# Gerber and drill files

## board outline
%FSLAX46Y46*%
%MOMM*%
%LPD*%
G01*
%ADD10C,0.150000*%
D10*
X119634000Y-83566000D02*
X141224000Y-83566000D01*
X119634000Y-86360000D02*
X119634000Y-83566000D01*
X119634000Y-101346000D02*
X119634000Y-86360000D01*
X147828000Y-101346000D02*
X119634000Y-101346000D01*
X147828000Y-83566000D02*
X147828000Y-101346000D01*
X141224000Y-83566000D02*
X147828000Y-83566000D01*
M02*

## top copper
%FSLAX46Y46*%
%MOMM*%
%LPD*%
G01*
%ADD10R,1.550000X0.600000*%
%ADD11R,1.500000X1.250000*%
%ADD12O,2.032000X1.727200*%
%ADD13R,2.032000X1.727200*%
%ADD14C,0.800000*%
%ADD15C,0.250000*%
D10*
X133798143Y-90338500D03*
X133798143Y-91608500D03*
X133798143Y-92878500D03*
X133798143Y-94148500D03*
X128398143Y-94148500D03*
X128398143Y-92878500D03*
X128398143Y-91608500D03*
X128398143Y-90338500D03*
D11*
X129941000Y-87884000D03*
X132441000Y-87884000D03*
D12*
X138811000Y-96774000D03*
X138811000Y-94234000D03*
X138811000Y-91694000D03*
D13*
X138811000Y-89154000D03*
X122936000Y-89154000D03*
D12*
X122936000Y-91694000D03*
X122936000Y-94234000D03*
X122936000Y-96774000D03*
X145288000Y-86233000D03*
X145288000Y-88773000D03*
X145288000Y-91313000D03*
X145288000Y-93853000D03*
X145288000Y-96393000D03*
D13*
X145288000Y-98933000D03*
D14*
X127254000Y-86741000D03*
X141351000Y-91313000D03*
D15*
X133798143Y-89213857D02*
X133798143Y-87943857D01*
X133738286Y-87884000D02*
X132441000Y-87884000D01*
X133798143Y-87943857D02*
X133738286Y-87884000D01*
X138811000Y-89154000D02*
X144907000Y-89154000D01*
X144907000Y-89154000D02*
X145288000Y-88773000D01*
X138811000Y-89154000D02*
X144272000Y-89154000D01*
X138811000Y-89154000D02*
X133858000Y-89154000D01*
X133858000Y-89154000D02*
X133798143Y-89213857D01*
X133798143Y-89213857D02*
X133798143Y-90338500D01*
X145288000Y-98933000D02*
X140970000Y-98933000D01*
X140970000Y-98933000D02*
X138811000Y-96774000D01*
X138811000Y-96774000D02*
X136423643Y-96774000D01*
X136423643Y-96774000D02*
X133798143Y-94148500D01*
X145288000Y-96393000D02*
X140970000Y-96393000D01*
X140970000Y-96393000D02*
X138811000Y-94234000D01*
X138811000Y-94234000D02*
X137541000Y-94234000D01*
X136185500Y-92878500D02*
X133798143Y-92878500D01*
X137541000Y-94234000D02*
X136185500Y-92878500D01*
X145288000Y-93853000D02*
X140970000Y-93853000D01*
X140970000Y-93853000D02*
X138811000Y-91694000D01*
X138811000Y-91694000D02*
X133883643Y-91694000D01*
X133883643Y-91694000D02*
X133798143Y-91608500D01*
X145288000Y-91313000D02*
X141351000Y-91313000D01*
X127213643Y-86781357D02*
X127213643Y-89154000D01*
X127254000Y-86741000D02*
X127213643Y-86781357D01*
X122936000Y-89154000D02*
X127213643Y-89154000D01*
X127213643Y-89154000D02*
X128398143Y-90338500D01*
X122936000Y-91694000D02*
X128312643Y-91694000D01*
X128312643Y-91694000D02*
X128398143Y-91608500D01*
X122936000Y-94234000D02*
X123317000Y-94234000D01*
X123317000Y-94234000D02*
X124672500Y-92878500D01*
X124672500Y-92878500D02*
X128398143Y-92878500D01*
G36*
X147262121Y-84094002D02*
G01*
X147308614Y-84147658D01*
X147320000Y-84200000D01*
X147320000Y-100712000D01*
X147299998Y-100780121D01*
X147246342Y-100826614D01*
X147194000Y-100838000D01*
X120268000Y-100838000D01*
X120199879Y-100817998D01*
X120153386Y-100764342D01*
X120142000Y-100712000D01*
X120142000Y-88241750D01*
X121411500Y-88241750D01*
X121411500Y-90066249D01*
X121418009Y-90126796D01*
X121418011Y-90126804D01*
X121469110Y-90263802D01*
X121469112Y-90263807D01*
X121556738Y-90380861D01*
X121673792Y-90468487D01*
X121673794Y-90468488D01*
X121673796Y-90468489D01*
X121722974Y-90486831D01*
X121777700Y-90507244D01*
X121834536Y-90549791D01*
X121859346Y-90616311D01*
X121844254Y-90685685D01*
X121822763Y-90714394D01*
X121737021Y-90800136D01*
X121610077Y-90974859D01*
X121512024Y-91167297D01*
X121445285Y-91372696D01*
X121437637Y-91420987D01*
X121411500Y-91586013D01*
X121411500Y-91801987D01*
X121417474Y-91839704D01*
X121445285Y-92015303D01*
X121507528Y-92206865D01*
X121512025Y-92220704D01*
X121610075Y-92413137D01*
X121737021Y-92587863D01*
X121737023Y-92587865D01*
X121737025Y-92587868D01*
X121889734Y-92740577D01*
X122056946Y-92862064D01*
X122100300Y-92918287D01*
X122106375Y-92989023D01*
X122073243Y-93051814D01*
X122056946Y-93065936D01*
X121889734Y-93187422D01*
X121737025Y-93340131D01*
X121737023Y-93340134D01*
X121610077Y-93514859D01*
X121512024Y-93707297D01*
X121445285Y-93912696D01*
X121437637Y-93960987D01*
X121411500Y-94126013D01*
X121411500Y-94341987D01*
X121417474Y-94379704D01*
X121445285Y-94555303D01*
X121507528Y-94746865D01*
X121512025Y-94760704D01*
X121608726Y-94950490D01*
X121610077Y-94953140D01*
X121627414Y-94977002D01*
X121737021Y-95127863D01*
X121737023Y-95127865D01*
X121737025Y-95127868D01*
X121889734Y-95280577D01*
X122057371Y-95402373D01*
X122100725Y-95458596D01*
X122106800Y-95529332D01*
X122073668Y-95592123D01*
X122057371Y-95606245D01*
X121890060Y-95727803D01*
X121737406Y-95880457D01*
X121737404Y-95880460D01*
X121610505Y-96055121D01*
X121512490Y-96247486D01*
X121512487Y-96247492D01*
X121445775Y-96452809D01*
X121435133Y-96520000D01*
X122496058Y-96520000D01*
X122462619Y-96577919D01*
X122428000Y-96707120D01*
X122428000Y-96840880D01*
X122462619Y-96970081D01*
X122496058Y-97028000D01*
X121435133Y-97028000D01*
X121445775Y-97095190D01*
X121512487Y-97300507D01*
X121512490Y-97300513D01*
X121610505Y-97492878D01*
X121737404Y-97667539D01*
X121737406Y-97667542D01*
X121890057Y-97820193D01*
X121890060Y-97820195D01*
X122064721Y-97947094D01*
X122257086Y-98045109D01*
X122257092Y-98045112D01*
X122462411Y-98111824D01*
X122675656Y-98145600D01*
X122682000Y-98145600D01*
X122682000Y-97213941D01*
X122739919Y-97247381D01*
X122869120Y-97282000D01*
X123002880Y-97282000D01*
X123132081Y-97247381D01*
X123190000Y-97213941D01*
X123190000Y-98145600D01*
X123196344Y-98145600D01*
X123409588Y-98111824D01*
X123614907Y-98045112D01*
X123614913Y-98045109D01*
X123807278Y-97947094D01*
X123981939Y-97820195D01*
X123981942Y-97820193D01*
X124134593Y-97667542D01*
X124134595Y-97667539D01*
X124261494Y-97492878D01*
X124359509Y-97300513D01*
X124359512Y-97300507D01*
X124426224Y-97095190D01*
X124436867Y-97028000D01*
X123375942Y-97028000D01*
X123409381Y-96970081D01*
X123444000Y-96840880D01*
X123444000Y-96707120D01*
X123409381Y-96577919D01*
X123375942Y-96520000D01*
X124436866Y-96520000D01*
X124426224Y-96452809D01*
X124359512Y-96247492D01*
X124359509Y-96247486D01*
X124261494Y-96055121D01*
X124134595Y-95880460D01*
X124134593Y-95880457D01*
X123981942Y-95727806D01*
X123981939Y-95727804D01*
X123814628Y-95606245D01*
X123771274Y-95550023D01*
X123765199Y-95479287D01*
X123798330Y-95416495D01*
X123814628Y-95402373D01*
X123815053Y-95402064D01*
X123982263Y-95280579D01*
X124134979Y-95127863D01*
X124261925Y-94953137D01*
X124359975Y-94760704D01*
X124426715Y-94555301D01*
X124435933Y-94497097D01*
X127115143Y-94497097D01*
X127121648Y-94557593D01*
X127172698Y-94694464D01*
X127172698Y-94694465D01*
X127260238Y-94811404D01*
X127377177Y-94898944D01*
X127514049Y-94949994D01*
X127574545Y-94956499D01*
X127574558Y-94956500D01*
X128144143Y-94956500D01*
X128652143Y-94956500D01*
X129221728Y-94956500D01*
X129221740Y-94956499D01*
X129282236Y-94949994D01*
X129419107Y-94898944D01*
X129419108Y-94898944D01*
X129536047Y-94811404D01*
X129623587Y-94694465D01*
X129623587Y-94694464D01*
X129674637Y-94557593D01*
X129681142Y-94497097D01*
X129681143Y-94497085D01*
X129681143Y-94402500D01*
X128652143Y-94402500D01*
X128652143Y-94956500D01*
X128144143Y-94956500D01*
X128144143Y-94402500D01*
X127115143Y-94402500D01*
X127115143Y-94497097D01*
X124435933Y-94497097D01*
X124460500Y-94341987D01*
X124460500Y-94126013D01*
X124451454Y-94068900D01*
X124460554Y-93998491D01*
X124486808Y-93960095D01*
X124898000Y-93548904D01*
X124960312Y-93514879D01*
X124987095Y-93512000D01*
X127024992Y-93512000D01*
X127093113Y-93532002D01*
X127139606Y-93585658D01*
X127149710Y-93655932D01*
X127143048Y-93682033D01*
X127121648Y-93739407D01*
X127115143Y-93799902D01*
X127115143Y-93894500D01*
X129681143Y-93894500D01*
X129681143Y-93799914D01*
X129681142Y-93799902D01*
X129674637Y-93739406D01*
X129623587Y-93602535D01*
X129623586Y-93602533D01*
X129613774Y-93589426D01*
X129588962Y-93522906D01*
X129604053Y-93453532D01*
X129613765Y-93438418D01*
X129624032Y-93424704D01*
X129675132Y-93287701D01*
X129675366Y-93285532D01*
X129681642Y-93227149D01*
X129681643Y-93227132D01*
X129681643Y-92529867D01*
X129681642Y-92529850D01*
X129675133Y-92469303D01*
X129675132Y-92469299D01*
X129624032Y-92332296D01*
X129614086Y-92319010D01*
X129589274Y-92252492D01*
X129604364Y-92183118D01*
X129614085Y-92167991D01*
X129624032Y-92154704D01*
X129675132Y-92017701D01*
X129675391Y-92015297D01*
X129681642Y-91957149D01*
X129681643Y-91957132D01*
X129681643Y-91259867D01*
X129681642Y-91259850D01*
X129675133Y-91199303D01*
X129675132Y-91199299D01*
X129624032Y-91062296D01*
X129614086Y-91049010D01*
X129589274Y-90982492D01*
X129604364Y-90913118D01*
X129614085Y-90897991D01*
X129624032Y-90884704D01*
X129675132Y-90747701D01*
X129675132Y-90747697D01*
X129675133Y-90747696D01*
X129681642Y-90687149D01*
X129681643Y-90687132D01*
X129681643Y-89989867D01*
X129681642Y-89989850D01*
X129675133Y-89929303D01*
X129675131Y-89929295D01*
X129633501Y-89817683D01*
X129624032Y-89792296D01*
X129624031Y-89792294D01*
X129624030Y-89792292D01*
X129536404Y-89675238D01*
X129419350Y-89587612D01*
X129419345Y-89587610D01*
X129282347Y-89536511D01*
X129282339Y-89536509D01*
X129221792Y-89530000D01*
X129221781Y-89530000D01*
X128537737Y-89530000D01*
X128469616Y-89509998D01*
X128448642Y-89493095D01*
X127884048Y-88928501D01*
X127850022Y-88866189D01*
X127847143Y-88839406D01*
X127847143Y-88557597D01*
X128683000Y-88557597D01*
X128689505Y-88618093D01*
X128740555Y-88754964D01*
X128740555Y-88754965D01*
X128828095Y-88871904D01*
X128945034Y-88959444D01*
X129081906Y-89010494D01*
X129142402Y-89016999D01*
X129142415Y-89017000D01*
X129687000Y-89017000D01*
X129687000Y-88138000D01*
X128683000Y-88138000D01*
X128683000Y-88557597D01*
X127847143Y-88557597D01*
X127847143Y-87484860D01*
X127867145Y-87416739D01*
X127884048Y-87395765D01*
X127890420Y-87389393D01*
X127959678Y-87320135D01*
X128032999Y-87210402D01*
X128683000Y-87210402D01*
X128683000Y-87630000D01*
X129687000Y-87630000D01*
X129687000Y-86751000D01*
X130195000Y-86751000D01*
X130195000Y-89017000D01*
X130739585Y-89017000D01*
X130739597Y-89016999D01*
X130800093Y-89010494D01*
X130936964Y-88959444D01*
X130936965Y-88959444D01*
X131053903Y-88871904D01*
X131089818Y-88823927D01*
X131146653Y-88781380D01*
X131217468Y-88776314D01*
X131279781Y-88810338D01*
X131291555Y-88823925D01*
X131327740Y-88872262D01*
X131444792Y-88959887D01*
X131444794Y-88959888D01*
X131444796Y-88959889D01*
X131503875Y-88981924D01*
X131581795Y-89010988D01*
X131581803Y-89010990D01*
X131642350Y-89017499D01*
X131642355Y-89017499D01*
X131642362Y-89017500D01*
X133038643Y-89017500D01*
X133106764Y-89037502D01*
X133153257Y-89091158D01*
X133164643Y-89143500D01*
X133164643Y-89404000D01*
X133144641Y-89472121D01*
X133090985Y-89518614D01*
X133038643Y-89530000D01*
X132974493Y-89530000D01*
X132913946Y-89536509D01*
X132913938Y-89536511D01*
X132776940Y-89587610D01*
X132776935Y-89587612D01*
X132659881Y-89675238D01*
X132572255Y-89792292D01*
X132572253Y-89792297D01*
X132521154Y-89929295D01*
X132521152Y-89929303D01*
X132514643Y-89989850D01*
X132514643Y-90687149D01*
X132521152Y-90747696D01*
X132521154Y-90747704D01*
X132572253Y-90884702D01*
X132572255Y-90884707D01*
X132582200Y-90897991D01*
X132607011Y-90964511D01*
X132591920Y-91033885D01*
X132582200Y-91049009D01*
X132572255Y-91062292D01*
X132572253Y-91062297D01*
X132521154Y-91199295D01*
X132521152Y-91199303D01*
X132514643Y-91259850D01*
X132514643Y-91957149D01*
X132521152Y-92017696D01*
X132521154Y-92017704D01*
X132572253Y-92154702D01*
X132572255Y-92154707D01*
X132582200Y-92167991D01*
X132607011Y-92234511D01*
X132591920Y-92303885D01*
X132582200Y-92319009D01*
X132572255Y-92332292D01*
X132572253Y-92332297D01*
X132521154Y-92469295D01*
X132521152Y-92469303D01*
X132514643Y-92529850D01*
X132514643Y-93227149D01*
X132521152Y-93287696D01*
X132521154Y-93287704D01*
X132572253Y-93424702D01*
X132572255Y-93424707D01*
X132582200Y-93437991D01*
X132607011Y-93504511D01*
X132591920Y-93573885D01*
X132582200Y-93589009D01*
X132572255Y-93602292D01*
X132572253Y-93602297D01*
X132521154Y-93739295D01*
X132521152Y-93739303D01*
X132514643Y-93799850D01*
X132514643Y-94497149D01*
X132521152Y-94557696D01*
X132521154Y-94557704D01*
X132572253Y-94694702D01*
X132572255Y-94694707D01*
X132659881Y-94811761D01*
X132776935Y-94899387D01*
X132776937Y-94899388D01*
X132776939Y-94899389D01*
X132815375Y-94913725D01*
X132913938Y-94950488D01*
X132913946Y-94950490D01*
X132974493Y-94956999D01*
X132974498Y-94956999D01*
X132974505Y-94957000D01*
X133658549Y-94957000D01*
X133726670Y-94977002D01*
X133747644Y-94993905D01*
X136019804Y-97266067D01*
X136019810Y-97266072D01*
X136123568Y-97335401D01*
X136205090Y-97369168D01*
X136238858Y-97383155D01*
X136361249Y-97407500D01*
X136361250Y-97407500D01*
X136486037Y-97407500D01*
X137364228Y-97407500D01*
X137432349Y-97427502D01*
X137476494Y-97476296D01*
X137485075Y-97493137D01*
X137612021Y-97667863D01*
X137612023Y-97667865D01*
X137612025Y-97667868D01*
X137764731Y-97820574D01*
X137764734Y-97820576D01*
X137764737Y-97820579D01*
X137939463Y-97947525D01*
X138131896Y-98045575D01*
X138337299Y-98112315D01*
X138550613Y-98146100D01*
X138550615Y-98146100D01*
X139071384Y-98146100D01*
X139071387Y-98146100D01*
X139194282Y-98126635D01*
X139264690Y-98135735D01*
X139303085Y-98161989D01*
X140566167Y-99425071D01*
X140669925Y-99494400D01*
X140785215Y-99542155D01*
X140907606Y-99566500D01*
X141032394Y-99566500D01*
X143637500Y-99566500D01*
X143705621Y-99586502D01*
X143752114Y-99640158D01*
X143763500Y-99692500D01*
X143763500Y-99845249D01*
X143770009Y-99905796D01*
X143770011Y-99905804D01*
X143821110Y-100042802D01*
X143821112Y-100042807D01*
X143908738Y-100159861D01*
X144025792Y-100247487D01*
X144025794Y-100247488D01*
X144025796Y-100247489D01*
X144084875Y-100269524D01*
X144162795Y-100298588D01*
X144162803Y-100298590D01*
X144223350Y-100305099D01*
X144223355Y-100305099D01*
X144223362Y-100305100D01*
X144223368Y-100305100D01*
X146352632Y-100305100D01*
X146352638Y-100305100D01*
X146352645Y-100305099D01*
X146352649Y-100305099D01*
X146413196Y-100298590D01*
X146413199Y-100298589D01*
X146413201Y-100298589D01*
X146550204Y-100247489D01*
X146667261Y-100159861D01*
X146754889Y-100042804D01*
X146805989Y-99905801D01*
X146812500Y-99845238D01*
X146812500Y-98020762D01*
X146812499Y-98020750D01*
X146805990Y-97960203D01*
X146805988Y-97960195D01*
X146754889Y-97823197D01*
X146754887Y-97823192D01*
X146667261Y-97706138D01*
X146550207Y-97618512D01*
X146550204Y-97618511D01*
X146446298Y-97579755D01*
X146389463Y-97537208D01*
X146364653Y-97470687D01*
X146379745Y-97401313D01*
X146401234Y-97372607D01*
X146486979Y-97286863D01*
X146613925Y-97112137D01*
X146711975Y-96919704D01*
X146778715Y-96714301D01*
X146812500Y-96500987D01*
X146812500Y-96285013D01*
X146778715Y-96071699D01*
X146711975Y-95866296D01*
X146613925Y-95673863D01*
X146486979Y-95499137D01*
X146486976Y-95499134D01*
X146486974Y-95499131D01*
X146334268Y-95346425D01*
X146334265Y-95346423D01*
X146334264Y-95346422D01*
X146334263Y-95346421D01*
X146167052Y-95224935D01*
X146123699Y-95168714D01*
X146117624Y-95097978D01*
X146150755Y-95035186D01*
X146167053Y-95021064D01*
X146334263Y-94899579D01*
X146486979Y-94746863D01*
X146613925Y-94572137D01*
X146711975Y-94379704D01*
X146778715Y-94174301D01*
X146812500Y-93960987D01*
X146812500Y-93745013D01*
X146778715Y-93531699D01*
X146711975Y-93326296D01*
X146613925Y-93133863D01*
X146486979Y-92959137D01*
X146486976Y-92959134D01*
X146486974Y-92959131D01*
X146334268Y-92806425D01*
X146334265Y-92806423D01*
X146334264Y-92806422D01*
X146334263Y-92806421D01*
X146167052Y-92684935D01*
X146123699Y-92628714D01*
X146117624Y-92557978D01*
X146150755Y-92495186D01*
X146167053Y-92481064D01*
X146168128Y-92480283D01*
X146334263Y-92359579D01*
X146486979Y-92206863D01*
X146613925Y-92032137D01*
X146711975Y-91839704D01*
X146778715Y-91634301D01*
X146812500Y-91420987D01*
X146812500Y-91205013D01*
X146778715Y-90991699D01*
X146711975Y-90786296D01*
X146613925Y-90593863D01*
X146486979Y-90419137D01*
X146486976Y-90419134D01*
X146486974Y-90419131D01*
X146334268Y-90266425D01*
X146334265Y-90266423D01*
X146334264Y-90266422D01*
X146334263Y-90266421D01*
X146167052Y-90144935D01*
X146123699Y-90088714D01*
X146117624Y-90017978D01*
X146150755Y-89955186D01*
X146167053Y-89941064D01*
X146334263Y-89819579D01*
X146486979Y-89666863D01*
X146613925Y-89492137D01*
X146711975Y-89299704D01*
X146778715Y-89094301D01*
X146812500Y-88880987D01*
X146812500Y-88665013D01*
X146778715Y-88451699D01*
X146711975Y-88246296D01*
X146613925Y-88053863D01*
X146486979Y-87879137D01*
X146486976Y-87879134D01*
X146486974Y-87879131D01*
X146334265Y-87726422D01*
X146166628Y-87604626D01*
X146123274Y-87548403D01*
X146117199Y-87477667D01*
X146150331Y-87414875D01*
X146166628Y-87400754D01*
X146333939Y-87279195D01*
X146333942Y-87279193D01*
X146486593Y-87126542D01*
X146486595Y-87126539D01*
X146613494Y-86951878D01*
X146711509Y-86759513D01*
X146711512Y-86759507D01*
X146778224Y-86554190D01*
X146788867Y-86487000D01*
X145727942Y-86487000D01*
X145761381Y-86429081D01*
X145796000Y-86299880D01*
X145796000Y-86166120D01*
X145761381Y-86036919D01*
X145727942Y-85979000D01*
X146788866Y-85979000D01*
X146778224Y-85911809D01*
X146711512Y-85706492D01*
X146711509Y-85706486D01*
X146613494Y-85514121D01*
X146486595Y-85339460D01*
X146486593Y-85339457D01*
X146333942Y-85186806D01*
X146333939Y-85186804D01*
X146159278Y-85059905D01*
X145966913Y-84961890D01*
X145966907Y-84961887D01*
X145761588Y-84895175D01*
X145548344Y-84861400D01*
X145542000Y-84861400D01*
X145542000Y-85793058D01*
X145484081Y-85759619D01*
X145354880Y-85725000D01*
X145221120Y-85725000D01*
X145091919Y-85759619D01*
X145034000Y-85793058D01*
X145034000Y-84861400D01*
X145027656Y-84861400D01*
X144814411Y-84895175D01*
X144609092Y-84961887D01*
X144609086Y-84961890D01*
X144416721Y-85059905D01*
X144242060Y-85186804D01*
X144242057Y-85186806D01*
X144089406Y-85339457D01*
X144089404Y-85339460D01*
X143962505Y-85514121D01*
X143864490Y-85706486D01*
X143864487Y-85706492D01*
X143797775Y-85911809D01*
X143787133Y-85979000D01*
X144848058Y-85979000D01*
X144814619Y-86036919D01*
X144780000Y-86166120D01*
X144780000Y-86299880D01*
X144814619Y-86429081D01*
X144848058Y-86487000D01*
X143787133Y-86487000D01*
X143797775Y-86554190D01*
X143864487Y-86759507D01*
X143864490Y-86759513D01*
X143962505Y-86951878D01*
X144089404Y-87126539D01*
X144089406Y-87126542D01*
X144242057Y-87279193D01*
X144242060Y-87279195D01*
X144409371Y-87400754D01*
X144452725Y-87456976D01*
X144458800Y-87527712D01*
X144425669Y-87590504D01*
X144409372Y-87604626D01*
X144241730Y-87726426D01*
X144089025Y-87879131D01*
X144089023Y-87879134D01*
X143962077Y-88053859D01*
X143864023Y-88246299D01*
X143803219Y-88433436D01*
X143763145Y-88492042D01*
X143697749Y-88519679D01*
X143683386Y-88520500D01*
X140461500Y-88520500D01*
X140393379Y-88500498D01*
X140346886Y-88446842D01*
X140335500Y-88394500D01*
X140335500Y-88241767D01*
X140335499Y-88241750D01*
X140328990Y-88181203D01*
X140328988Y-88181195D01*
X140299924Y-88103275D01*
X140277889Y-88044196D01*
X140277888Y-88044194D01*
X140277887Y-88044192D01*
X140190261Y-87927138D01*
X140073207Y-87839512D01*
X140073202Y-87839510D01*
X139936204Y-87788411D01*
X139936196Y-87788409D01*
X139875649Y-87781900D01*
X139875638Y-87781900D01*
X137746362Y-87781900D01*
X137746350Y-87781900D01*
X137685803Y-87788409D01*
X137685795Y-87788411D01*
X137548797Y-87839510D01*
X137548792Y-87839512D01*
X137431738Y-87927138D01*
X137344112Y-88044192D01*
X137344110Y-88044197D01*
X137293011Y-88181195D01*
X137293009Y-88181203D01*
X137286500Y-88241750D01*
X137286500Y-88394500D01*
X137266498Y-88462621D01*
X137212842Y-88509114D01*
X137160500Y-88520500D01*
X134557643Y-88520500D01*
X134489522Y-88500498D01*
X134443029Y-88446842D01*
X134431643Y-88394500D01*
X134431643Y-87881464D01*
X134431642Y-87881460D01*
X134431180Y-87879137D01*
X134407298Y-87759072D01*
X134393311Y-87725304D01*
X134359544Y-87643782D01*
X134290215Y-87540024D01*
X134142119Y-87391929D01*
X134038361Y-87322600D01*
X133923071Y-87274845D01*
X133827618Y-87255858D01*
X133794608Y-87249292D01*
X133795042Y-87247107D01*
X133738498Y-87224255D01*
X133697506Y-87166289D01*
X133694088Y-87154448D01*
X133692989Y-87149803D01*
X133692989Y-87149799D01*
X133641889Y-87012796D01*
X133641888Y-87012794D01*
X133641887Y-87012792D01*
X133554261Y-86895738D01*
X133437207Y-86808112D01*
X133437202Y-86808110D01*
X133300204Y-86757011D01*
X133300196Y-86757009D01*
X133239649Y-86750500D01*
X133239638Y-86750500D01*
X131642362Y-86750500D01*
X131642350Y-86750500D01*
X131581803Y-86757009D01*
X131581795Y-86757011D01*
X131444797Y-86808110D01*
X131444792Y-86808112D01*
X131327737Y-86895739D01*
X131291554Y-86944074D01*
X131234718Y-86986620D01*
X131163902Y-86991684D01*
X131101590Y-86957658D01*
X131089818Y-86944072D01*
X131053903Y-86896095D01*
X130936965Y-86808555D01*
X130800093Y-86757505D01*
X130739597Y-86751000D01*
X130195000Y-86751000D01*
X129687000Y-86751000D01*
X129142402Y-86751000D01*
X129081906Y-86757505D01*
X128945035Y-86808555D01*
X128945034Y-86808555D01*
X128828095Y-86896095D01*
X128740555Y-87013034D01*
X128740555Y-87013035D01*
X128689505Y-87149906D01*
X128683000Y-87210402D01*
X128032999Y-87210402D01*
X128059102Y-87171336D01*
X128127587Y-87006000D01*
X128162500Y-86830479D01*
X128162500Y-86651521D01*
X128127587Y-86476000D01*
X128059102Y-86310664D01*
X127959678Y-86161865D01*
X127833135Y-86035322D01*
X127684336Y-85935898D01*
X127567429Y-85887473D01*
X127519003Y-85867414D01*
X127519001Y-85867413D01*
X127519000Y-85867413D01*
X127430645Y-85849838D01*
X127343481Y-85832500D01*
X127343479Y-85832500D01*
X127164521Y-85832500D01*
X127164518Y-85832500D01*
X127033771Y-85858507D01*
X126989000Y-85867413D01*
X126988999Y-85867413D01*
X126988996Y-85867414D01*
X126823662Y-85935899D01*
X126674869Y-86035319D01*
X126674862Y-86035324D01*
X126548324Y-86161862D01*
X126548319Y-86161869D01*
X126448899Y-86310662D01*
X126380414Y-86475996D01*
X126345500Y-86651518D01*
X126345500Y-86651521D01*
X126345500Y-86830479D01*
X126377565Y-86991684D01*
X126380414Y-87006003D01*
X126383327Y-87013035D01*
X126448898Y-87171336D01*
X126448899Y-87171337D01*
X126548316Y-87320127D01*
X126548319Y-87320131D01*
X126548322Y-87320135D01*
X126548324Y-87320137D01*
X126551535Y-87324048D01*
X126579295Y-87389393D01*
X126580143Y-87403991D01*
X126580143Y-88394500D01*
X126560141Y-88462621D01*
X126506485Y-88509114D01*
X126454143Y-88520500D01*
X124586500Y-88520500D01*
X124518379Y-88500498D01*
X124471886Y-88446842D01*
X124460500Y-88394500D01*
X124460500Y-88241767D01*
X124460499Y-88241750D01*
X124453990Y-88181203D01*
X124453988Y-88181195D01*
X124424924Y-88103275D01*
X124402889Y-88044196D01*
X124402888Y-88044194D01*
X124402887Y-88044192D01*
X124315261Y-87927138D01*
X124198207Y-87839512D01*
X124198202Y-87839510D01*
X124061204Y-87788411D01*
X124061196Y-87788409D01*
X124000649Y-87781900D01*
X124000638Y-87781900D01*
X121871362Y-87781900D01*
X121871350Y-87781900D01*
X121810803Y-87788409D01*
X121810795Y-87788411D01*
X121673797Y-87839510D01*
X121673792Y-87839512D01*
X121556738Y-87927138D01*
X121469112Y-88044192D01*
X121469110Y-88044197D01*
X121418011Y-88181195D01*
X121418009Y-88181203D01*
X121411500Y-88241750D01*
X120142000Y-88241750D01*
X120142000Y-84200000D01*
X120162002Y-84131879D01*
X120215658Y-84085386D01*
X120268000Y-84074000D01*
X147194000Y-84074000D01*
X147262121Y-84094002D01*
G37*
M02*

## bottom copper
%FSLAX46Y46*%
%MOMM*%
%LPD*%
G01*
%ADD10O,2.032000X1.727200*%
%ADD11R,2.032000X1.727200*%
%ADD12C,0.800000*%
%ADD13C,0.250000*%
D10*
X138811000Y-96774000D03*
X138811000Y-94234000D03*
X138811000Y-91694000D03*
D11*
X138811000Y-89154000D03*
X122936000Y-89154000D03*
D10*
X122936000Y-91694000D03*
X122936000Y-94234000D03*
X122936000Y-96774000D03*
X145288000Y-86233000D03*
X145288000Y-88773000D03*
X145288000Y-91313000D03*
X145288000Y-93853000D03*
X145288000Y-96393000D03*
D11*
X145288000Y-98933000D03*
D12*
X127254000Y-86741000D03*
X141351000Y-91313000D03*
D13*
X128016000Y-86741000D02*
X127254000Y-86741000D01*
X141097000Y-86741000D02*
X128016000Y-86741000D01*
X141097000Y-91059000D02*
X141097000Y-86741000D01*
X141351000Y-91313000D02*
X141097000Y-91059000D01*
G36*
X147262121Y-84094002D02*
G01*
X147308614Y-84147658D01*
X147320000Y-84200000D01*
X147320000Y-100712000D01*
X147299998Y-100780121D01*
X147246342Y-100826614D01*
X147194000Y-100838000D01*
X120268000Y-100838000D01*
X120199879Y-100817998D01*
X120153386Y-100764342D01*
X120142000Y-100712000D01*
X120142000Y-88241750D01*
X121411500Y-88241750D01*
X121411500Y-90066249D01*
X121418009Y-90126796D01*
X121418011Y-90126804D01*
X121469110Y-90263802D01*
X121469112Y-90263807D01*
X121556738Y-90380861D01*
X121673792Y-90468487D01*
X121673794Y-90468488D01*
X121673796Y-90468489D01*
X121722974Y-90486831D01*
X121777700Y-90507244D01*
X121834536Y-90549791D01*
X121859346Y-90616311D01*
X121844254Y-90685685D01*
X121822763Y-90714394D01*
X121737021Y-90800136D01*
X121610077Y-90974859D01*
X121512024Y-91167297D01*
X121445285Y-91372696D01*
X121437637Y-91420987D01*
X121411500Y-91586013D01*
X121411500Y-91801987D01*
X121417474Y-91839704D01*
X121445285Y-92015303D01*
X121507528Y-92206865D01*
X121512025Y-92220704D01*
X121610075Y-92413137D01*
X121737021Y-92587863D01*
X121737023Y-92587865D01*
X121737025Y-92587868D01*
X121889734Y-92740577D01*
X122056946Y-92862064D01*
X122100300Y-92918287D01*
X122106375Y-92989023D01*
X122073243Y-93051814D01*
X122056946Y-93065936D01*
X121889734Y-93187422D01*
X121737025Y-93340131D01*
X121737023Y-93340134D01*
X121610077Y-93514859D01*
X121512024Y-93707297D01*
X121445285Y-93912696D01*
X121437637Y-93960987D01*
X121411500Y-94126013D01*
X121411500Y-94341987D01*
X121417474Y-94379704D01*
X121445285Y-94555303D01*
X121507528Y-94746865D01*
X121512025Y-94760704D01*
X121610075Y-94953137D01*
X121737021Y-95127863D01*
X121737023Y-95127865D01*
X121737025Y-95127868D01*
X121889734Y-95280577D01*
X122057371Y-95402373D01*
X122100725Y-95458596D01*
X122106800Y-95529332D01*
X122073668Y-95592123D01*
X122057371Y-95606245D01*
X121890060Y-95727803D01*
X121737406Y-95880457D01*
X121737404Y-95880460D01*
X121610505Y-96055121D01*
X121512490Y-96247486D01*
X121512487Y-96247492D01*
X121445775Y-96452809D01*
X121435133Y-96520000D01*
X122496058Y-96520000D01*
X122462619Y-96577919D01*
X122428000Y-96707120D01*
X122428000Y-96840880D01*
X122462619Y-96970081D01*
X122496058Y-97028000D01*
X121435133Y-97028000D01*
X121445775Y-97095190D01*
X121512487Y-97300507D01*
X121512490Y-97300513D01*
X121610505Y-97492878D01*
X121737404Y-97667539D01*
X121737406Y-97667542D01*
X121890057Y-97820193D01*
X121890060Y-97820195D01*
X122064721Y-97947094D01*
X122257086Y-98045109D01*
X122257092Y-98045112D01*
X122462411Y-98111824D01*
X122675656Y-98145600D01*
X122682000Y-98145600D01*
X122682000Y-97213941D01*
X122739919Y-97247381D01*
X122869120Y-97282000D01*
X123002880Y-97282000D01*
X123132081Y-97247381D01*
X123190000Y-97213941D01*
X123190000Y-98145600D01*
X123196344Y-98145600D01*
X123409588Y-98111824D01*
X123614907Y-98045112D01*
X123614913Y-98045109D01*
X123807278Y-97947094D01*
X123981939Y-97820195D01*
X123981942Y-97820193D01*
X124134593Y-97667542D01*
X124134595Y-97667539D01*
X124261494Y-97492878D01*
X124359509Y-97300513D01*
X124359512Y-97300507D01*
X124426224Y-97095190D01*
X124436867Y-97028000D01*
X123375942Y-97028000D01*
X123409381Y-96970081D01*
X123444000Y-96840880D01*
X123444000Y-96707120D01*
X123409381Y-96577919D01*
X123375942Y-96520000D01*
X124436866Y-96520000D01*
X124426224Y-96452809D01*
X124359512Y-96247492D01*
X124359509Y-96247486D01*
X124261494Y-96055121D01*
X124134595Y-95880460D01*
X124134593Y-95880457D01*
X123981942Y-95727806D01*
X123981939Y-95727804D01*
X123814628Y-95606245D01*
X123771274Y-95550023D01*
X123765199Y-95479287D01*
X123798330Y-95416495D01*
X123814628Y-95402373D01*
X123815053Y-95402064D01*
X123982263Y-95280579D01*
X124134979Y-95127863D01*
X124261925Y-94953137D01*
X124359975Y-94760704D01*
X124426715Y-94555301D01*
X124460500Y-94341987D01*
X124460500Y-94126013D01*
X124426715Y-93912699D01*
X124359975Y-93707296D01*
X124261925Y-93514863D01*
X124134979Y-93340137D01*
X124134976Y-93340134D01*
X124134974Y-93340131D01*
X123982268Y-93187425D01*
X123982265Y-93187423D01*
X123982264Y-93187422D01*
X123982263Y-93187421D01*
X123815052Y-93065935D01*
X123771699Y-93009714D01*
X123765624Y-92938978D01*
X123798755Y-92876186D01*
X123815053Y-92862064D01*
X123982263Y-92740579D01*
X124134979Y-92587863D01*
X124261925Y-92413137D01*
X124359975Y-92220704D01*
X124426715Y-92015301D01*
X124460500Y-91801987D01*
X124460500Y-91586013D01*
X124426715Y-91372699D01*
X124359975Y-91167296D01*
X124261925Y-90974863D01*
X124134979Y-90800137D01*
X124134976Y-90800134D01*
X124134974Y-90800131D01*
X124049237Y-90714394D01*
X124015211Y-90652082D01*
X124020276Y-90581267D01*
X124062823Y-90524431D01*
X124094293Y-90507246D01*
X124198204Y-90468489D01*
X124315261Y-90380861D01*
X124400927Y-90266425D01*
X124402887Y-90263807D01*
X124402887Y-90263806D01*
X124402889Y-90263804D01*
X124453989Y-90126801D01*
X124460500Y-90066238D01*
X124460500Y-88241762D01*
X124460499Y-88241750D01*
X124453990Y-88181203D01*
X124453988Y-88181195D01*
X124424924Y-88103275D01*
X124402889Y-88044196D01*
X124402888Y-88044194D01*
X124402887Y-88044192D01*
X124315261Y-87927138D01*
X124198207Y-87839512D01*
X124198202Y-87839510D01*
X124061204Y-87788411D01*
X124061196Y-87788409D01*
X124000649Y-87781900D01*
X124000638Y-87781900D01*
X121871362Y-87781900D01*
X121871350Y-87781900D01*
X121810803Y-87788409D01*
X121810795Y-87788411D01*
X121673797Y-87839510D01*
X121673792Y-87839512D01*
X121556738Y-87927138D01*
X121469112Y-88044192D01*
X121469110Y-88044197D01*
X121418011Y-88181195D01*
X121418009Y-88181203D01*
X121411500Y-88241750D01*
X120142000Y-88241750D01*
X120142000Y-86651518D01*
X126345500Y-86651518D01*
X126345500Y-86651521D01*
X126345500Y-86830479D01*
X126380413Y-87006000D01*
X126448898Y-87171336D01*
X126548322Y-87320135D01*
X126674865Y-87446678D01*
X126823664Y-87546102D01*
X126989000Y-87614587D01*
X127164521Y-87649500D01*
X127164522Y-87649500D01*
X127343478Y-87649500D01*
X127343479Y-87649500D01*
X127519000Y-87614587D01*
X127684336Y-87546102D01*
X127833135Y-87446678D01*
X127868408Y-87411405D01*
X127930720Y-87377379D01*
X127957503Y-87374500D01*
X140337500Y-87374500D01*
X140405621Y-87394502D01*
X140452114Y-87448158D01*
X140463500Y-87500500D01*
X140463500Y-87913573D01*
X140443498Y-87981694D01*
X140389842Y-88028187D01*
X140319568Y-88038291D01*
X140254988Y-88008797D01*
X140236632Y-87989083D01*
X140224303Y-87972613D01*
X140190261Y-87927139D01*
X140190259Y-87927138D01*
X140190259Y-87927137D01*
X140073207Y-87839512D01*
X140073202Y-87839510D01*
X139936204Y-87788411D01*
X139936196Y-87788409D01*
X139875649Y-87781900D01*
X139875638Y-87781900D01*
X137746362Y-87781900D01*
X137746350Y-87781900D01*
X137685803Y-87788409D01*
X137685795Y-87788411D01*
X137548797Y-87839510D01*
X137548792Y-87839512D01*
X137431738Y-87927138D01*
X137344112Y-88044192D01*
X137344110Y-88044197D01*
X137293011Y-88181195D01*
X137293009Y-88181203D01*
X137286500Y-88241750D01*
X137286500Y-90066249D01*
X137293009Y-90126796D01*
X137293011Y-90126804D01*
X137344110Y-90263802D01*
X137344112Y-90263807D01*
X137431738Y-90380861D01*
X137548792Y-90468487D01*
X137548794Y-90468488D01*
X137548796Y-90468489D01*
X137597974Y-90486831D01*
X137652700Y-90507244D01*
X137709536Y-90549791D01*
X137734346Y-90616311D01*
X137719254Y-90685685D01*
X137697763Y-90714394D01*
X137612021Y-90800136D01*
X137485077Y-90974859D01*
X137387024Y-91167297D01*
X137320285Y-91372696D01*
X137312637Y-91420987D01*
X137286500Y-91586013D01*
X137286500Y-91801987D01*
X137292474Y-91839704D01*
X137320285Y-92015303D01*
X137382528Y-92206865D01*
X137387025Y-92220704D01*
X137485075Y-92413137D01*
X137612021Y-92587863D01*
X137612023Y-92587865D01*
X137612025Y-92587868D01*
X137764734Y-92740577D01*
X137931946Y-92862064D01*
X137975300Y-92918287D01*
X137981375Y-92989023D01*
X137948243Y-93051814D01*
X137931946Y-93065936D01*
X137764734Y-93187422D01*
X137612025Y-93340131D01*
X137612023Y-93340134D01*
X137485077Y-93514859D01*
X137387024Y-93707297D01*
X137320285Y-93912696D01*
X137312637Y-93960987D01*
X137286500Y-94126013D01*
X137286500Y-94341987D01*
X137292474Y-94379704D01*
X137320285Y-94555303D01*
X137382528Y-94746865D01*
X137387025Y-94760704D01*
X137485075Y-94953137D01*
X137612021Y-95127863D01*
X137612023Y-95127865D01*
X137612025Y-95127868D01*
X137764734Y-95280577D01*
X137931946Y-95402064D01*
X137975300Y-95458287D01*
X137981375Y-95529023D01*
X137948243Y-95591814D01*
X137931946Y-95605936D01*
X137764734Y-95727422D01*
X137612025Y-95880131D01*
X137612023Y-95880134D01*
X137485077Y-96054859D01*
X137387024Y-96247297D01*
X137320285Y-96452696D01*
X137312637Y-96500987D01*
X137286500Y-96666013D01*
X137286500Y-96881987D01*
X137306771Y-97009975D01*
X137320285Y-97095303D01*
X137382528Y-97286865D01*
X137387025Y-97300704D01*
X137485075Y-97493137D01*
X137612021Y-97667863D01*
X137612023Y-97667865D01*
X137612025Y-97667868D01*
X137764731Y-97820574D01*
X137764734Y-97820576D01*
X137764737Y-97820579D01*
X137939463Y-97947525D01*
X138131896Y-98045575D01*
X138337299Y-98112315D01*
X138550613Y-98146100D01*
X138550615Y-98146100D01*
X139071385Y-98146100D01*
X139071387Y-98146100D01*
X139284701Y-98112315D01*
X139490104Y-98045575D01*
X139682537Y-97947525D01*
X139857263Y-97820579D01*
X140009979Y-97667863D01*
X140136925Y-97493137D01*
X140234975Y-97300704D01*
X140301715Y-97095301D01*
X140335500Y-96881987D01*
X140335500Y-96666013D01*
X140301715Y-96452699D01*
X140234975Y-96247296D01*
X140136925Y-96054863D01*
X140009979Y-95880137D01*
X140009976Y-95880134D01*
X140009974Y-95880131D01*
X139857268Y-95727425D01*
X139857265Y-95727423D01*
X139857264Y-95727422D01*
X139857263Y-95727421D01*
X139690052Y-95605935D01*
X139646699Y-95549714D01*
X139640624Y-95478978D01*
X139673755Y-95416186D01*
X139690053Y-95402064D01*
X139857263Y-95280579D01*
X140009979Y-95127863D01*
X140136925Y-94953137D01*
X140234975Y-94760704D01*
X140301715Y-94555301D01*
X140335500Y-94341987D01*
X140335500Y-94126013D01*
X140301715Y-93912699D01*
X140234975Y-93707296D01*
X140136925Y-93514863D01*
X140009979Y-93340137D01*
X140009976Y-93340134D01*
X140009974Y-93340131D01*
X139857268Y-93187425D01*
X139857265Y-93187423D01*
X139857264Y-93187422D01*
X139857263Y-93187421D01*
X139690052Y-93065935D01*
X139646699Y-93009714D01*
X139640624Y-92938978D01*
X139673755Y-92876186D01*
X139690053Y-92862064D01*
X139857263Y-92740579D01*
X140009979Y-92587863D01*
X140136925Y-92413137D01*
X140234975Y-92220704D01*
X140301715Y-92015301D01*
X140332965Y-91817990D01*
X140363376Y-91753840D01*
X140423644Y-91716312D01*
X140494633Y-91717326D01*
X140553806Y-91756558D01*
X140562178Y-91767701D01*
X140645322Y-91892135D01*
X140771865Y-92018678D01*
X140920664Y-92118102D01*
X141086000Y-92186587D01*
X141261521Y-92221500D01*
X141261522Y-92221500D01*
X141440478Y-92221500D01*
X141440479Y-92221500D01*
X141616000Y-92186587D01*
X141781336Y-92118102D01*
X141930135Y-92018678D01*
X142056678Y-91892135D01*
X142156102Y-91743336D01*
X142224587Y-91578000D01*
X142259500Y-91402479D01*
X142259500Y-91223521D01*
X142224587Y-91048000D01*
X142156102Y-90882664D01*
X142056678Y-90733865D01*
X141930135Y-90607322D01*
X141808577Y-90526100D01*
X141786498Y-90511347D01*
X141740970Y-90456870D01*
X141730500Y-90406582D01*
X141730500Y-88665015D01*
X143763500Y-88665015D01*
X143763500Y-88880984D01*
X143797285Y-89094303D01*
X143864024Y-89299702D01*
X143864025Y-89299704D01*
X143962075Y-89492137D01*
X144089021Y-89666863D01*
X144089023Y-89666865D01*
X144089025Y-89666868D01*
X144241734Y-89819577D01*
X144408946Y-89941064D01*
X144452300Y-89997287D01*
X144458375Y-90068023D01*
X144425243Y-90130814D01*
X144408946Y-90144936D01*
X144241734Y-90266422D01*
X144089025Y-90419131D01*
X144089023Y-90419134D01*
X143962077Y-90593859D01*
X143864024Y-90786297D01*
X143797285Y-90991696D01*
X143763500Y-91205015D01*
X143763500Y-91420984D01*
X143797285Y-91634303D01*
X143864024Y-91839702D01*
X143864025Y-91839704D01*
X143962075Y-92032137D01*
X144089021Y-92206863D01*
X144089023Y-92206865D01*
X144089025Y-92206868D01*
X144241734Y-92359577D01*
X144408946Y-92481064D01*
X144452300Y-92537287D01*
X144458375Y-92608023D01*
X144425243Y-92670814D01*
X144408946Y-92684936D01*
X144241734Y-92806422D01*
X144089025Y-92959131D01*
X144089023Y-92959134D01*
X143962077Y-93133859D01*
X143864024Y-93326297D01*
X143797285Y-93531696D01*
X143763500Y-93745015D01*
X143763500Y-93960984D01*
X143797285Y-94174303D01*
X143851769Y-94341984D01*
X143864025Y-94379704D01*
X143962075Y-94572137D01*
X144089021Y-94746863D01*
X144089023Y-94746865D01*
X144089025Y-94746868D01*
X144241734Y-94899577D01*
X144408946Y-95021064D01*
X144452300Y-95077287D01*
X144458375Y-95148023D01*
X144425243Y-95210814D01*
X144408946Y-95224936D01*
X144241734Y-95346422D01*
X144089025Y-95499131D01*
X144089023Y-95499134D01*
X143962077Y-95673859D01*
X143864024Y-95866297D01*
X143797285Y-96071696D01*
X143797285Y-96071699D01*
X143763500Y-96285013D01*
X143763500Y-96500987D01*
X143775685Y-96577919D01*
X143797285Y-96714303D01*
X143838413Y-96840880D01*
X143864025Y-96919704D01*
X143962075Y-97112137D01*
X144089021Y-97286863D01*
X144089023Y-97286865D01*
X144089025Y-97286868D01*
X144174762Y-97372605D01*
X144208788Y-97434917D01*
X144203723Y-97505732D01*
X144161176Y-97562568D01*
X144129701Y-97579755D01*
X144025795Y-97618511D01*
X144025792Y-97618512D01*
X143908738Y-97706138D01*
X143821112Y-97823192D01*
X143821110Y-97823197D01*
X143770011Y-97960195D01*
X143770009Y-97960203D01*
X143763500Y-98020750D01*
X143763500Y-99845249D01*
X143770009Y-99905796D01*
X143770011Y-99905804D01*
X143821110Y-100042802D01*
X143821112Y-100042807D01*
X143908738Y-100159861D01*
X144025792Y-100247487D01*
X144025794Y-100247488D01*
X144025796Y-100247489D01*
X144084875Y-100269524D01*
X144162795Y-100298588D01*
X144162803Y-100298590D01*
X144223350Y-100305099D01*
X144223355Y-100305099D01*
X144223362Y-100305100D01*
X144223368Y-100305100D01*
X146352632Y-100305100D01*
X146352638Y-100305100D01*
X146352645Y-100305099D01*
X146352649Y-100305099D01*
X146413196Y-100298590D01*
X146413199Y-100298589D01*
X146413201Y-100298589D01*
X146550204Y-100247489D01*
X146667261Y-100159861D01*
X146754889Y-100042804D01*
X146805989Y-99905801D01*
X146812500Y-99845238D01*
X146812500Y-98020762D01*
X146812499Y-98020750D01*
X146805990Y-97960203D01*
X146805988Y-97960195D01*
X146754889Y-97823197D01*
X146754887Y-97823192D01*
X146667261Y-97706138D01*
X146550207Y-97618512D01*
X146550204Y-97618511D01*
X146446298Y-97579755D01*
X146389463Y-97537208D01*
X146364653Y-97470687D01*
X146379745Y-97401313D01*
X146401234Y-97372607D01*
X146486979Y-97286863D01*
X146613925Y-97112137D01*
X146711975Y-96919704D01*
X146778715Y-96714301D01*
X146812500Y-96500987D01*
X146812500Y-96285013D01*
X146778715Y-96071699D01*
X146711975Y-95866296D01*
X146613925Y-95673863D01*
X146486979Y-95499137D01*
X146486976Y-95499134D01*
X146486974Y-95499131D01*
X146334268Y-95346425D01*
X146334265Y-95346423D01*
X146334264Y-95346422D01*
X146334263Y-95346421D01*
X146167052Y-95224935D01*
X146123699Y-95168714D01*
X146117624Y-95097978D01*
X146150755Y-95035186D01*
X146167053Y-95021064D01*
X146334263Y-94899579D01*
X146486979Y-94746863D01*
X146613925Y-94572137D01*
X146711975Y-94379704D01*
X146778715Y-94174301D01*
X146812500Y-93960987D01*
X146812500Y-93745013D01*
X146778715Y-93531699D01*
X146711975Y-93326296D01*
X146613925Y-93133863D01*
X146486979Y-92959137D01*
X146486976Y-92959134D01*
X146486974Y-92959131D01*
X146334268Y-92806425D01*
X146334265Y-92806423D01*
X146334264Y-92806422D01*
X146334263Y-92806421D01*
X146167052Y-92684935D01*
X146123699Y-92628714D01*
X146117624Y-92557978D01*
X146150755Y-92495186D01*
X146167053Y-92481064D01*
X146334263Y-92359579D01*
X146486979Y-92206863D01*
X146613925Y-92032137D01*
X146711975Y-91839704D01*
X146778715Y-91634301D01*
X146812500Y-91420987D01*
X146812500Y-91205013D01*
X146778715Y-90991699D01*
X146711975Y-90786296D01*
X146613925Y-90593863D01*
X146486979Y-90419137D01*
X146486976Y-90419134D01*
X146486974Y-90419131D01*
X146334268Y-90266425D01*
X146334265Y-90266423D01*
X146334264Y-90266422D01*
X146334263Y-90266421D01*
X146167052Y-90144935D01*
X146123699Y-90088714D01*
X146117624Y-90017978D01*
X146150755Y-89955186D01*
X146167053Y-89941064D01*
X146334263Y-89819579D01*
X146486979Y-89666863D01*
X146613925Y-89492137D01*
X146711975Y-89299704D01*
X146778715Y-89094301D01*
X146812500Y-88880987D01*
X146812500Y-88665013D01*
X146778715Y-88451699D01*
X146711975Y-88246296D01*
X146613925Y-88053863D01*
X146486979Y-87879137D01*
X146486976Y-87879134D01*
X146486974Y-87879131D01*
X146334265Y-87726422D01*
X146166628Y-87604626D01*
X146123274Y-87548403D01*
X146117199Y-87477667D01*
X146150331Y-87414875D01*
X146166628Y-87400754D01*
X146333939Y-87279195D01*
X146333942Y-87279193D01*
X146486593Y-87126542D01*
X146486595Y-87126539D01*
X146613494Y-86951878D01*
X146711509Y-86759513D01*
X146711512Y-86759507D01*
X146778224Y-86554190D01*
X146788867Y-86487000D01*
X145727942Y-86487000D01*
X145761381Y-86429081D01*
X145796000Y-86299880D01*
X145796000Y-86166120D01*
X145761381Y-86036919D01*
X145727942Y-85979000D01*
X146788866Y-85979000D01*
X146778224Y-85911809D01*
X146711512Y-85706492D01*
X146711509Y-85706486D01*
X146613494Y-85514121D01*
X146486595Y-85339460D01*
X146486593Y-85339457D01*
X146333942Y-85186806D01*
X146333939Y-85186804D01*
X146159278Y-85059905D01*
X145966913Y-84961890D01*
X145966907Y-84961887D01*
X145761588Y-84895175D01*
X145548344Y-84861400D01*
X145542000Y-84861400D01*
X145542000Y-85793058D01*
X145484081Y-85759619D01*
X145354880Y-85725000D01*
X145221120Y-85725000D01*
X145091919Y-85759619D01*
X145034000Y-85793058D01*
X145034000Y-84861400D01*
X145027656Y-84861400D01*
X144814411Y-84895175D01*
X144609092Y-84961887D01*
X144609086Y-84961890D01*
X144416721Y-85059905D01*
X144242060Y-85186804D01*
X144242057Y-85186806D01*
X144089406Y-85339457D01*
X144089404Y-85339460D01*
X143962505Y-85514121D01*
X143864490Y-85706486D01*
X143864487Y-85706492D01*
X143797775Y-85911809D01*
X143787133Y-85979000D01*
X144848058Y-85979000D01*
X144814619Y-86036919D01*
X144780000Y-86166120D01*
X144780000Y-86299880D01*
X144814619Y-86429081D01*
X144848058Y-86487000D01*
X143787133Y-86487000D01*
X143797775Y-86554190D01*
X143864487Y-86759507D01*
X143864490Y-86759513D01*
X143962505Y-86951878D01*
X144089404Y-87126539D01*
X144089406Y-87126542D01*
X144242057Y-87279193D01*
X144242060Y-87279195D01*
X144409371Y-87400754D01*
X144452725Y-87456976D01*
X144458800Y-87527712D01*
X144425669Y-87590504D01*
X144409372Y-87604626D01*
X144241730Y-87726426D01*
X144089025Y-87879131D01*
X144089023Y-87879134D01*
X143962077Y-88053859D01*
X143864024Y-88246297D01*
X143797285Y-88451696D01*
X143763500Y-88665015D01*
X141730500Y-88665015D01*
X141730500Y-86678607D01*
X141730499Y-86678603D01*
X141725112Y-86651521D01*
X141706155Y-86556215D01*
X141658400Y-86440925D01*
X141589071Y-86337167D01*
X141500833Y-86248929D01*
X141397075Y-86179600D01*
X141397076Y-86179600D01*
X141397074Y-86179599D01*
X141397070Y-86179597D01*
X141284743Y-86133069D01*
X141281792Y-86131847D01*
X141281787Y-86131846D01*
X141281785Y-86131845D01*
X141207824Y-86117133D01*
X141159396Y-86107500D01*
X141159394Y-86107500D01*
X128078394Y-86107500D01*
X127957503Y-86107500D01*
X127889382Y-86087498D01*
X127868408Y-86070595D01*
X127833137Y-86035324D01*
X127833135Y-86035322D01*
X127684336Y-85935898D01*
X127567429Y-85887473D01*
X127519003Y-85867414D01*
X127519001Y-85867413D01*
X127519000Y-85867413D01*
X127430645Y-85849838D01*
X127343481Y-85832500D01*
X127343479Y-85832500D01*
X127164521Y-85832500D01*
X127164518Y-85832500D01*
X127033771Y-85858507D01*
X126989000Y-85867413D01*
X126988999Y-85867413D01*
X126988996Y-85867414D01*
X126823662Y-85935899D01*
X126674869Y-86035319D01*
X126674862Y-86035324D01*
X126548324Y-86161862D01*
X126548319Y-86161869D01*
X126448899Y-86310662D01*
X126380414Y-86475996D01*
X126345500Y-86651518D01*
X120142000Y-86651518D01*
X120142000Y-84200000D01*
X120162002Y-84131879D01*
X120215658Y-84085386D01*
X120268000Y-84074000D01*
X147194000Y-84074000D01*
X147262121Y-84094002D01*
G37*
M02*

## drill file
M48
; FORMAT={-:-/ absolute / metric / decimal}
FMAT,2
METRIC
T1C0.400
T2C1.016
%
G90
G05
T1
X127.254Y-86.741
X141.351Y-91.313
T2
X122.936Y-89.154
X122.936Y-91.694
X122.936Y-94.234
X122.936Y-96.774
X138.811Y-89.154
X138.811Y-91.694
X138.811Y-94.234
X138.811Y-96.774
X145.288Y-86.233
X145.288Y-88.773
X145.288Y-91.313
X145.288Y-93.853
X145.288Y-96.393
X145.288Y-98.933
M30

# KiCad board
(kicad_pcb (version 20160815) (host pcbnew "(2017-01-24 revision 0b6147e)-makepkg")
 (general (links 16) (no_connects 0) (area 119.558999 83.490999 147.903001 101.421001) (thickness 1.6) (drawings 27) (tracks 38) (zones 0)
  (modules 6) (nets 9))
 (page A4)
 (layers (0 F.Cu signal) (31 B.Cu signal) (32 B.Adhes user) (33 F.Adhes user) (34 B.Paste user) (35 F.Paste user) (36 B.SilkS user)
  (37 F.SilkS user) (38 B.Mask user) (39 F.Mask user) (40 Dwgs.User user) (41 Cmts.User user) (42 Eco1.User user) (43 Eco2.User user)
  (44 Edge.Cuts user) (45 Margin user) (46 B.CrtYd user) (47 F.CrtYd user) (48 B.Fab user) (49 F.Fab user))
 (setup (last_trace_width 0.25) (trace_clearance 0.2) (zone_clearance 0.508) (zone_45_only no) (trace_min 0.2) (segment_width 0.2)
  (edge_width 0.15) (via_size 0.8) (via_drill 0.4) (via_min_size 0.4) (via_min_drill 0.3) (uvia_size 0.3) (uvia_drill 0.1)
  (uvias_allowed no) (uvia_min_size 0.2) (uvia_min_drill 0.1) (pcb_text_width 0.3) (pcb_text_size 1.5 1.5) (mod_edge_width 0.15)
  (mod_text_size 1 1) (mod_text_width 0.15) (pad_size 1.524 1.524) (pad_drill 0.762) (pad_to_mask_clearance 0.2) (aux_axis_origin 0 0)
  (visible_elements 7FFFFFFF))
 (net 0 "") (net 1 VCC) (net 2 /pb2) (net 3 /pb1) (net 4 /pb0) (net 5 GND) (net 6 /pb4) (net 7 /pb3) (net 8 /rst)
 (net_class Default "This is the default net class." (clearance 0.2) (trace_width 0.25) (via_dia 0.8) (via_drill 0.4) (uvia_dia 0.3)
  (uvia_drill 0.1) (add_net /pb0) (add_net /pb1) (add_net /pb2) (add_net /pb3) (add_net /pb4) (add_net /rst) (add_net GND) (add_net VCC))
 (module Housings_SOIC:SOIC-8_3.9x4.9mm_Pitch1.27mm (layer F.Cu) (at 131.098143 92.2435)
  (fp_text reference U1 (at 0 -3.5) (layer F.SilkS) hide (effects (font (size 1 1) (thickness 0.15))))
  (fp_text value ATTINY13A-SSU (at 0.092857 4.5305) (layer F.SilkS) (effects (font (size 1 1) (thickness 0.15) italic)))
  (pad 8 smd rect (at 2.7 -1.905) (size 1.55 0.6) (layers F.Cu F.Paste F.Mask) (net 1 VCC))
  (pad 7 smd rect (at 2.7 -0.635) (size 1.55 0.6) (layers F.Cu F.Paste F.Mask) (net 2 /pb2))
  (pad 6 smd rect (at 2.7 0.635) (size 1.55 0.6) (layers F.Cu F.Paste F.Mask) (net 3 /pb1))
  (pad 5 smd rect (at 2.7 1.905) (size 1.55 0.6) (layers F.Cu F.Paste F.Mask) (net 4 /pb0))
  (pad 4 smd rect (at -2.7 1.905) (size 1.55 0.6) (layers F.Cu F.Paste F.Mask) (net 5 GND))
  (pad 3 smd rect (at -2.7 0.635) (size 1.55 0.6) (layers F.Cu F.Paste F.Mask) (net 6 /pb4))
  (pad 2 smd rect (at -2.7 -0.635) (size 1.55 0.6) (layers F.Cu F.Paste F.Mask) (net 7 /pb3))
  (pad 1 smd rect (at -2.7 -1.905) (size 1.55 0.6) (layers F.Cu F.Paste F.Mask) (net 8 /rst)))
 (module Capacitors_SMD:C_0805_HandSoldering (layer F.Cu) (at 131.191 87.884 180)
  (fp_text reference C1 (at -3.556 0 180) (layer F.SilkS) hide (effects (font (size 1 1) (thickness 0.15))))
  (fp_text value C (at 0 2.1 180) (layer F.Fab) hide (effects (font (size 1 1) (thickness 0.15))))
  (pad 2 smd rect (at 1.25 0 180) (size 1.5 1.25) (layers F.Cu F.Paste F.Mask) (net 5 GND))
  (pad 1 smd rect (at -1.25 0 180) (size 1.5 1.25) (layers F.Cu F.Paste F.Mask) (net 1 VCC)))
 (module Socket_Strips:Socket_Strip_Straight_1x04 (layer F.Cu) (at 138.811 89.154 270)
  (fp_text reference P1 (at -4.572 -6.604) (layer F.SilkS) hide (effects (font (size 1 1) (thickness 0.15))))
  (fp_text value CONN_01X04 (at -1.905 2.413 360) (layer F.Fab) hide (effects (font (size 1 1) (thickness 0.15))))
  (pad 4 thru_hole oval (at 7.62 0 270) (size 1.7272 2.032) (drill 1.016) (layers *.Cu *.Mask) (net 4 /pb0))
  (pad 3 thru_hole oval (at 5.08 0 270) (size 1.7272 2.032) (drill 1.016) (layers *.Cu *.Mask) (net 3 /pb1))
  (pad 2 thru_hole oval (at 2.54 0 270) (size 1.7272 2.032) (drill 1.016) (layers *.Cu *.Mask) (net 2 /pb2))
  (pad 1 thru_hole rect (at 0 0 270) (size 1.7272 2.032) (drill 1.016) (layers *.Cu *.Mask) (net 1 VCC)))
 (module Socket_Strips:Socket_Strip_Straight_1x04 (layer F.Cu) (at 122.936 89.154 270)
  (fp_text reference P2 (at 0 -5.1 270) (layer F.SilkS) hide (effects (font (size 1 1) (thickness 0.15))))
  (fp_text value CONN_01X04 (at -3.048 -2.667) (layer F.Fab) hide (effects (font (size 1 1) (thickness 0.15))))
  (pad 1 thru_hole rect (at 0 0 270) (size 1.7272 2.032) (drill 1.016) (layers *.Cu *.Mask) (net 8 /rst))
  (pad 2 thru_hole oval (at 2.54 0 270) (size 1.7272 2.032) (drill 1.016) (layers *.Cu *.Mask) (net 7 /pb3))
  (pad 3 thru_hole oval (at 5.08 0 270) (size 1.7272 2.032) (drill 1.016) (layers *.Cu *.Mask) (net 6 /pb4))
  (pad 4 thru_hole oval (at 7.62 0 270) (size 1.7272 2.032) (drill 1.016) (layers *.Cu *.Mask) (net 5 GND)))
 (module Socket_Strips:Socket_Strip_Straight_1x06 (layer F.Cu) (at 145.288 98.933 90)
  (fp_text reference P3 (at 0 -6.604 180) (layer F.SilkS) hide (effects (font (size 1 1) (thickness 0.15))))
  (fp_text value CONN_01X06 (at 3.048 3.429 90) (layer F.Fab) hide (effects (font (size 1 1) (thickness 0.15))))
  (pad 6 thru_hole oval (at 12.7 0 90) (size 1.7272 2.032) (drill 1.016) (layers *.Cu *.Mask) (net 5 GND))
  (pad 5 thru_hole oval (at 10.16 0 90) (size 1.7272 2.032) (drill 1.016) (layers *.Cu *.Mask) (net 1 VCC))
  (pad 4 thru_hole oval (at 7.62 0 90) (size 1.7272 2.032) (drill 1.016) (layers *.Cu *.Mask) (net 8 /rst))
  (pad 3 thru_hole oval (at 5.08 0 90) (size 1.7272 2.032) (drill 1.016) (layers *.Cu *.Mask) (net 2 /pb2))
  (pad 2 thru_hole oval (at 2.54 0 90) (size 1.7272 2.032) (drill 1.016) (layers *.Cu *.Mask) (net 3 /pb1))
  (pad 1 thru_hole rect (at 0 0 90) (size 1.7272 2.032) (drill 1.016) (layers *.Cu *.Mask) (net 4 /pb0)))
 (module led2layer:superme (layer B.Cu) (at 129.286 96.52 180)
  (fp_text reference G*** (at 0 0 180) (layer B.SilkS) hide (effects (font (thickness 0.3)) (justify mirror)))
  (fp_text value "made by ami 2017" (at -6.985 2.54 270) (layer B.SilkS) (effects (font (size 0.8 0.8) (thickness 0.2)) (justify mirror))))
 (gr_line (start 119.634 83.566) (end 141.224 83.566) (angle 90) (layer Edge.Cuts) (width 0.15))
 (gr_line (start 119.634 86.36) (end 119.634 83.566) (angle 90) (layer Edge.Cuts) (width 0.15))
 (gr_line (start 119.634 101.346) (end 119.634 86.36) (angle 90) (layer Edge.Cuts) (width 0.15))
 (gr_line (start 147.828 101.346) (end 119.634 101.346) (angle 90) (layer Edge.Cuts) (width 0.15))
 (gr_line (start 147.828 83.566) (end 147.828 101.346) (angle 90) (layer Edge.Cuts) (width 0.15))
 (gr_line (start 141.224 83.566) (end 147.828 83.566) (angle 90) (layer Edge.Cuts) (width 0.15))
 (segment (start 133.798143 89.213857) (end 133.798143 87.943857) (width 0.25) (layer F.Cu) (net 1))
 (segment (start 133.738286 87.884) (end 132.441 87.884) (width 0.25) (layer F.Cu) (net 1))
 (segment (start 133.798143 87.943857) (end 133.738286 87.884) (width 0.25) (layer F.Cu) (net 1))
 (segment (start 138.811 89.154) (end 144.907 89.154) (width 0.25) (layer F.Cu) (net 1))
 (segment (start 144.907 89.154) (end 145.288 88.773) (width 0.25) (layer F.Cu) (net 1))
 (segment (start 138.811 89.154) (end 144.272 89.154) (width 0.25) (layer F.Cu) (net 1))
 (segment (start 138.811 89.154) (end 133.858 89.154) (width 0.25) (layer F.Cu) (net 1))
 (segment (start 133.858 89.154) (end 133.798143 89.213857) (width 0.25) (layer F.Cu) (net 1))
 (segment (start 133.798143 89.213857) (end 133.798143 90.3385) (width 0.25) (layer F.Cu) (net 1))
 (segment (start 145.288 98.933) (end 140.97 98.933) (width 0.25) (layer F.Cu) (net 4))
 (segment (start 140.97 98.933) (end 138.811 96.774) (width 0.25) (layer F.Cu) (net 4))
 (segment (start 138.811 96.774) (end 136.423643 96.774) (width 0.25) (layer F.Cu) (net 4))
 (segment (start 136.423643 96.774) (end 133.798143 94.1485) (width 0.25) (layer F.Cu) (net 4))
 (segment (start 145.288 96.393) (end 140.97 96.393) (width 0.25) (layer F.Cu) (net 3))
 (segment (start 140.97 96.393) (end 138.811 94.234) (width 0.25) (layer F.Cu) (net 3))
 (segment (start 138.811 94.234) (end 137.541 94.234) (width 0.25) (layer F.Cu) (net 3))
 (segment (start 136.1855 92.8785) (end 133.798143 92.8785) (width 0.25) (layer F.Cu) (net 3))
 (segment (start 137.541 94.234) (end 136.1855 92.8785) (width 0.25) (layer F.Cu) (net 3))
 (segment (start 145.288 93.853) (end 140.97 93.853) (width 0.25) (layer F.Cu) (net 2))
 (segment (start 140.97 93.853) (end 138.811 91.694) (width 0.25) (layer F.Cu) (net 2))
 (segment (start 138.811 91.694) (end 133.883643 91.694) (width 0.25) (layer F.Cu) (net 2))
 (segment (start 133.883643 91.694) (end 133.798143 91.6085) (width 0.25) (layer F.Cu) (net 2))
 (segment (start 145.288 91.313) (end 141.351 91.313) (width 0.25) (layer F.Cu) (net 8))
 (segment (start 127.213643 86.781357) (end 127.213643 89.154) (width 0.25) (layer F.Cu) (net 8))
 (segment (start 127.254 86.741) (end 127.213643 86.781357) (width 0.25) (layer F.Cu) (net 8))
 (via (at 127.254 86.741) (size 0.8) (drill 0.4) (layers F.Cu B.Cu) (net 8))
 (segment (start 128.016 86.741) (end 127.254 86.741) (width 0.25) (layer B.Cu) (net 8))
 (segment (start 141.097 86.741) (end 128.016 86.741) (width 0.25) (layer B.Cu) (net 8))
 (segment (start 141.097 91.059) (end 141.097 86.741) (width 0.25) (layer B.Cu) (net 8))
 (segment (start 141.351 91.313) (end 141.097 91.059) (width 0.25) (layer B.Cu) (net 8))
 (via (at 141.351 91.313) (size 0.8) (drill 0.4) (layers F.Cu B.Cu) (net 8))
 (segment (start 122.936 89.154) (end 127.213643 89.154) (width 0.25) (layer F.Cu) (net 8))
 (segment (start 127.213643 89.154) (end 128.398143 90.3385) (width 0.25) (layer F.Cu) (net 8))
 (segment (start 122.936 91.694) (end 128.312643 91.694) (width 0.25) (layer F.Cu) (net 7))
 (segment (start 128.312643 91.694) (end 128.398143 91.6085) (width 0.25) (layer F.Cu) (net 7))
 (segment (start 122.936 94.234) (end 123.317 94.234) (width 0.25) (layer F.Cu) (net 6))
 (segment (start 123.317 94.234) (end 124.6725 92.8785) (width 0.25) (layer F.Cu) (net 6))
 (segment (start 124.6725 92.8785) (end 128.398143 92.8785) (width 0.25) (layer F.Cu) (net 6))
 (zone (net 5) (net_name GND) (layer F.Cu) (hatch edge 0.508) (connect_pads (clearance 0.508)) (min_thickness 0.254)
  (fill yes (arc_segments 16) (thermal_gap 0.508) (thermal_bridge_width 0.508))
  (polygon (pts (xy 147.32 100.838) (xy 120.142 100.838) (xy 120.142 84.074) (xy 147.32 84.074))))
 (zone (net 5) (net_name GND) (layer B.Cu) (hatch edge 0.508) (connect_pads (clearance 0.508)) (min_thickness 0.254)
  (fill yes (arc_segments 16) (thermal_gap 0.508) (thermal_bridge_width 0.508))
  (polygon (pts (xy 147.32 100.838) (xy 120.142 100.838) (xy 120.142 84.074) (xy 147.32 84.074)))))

